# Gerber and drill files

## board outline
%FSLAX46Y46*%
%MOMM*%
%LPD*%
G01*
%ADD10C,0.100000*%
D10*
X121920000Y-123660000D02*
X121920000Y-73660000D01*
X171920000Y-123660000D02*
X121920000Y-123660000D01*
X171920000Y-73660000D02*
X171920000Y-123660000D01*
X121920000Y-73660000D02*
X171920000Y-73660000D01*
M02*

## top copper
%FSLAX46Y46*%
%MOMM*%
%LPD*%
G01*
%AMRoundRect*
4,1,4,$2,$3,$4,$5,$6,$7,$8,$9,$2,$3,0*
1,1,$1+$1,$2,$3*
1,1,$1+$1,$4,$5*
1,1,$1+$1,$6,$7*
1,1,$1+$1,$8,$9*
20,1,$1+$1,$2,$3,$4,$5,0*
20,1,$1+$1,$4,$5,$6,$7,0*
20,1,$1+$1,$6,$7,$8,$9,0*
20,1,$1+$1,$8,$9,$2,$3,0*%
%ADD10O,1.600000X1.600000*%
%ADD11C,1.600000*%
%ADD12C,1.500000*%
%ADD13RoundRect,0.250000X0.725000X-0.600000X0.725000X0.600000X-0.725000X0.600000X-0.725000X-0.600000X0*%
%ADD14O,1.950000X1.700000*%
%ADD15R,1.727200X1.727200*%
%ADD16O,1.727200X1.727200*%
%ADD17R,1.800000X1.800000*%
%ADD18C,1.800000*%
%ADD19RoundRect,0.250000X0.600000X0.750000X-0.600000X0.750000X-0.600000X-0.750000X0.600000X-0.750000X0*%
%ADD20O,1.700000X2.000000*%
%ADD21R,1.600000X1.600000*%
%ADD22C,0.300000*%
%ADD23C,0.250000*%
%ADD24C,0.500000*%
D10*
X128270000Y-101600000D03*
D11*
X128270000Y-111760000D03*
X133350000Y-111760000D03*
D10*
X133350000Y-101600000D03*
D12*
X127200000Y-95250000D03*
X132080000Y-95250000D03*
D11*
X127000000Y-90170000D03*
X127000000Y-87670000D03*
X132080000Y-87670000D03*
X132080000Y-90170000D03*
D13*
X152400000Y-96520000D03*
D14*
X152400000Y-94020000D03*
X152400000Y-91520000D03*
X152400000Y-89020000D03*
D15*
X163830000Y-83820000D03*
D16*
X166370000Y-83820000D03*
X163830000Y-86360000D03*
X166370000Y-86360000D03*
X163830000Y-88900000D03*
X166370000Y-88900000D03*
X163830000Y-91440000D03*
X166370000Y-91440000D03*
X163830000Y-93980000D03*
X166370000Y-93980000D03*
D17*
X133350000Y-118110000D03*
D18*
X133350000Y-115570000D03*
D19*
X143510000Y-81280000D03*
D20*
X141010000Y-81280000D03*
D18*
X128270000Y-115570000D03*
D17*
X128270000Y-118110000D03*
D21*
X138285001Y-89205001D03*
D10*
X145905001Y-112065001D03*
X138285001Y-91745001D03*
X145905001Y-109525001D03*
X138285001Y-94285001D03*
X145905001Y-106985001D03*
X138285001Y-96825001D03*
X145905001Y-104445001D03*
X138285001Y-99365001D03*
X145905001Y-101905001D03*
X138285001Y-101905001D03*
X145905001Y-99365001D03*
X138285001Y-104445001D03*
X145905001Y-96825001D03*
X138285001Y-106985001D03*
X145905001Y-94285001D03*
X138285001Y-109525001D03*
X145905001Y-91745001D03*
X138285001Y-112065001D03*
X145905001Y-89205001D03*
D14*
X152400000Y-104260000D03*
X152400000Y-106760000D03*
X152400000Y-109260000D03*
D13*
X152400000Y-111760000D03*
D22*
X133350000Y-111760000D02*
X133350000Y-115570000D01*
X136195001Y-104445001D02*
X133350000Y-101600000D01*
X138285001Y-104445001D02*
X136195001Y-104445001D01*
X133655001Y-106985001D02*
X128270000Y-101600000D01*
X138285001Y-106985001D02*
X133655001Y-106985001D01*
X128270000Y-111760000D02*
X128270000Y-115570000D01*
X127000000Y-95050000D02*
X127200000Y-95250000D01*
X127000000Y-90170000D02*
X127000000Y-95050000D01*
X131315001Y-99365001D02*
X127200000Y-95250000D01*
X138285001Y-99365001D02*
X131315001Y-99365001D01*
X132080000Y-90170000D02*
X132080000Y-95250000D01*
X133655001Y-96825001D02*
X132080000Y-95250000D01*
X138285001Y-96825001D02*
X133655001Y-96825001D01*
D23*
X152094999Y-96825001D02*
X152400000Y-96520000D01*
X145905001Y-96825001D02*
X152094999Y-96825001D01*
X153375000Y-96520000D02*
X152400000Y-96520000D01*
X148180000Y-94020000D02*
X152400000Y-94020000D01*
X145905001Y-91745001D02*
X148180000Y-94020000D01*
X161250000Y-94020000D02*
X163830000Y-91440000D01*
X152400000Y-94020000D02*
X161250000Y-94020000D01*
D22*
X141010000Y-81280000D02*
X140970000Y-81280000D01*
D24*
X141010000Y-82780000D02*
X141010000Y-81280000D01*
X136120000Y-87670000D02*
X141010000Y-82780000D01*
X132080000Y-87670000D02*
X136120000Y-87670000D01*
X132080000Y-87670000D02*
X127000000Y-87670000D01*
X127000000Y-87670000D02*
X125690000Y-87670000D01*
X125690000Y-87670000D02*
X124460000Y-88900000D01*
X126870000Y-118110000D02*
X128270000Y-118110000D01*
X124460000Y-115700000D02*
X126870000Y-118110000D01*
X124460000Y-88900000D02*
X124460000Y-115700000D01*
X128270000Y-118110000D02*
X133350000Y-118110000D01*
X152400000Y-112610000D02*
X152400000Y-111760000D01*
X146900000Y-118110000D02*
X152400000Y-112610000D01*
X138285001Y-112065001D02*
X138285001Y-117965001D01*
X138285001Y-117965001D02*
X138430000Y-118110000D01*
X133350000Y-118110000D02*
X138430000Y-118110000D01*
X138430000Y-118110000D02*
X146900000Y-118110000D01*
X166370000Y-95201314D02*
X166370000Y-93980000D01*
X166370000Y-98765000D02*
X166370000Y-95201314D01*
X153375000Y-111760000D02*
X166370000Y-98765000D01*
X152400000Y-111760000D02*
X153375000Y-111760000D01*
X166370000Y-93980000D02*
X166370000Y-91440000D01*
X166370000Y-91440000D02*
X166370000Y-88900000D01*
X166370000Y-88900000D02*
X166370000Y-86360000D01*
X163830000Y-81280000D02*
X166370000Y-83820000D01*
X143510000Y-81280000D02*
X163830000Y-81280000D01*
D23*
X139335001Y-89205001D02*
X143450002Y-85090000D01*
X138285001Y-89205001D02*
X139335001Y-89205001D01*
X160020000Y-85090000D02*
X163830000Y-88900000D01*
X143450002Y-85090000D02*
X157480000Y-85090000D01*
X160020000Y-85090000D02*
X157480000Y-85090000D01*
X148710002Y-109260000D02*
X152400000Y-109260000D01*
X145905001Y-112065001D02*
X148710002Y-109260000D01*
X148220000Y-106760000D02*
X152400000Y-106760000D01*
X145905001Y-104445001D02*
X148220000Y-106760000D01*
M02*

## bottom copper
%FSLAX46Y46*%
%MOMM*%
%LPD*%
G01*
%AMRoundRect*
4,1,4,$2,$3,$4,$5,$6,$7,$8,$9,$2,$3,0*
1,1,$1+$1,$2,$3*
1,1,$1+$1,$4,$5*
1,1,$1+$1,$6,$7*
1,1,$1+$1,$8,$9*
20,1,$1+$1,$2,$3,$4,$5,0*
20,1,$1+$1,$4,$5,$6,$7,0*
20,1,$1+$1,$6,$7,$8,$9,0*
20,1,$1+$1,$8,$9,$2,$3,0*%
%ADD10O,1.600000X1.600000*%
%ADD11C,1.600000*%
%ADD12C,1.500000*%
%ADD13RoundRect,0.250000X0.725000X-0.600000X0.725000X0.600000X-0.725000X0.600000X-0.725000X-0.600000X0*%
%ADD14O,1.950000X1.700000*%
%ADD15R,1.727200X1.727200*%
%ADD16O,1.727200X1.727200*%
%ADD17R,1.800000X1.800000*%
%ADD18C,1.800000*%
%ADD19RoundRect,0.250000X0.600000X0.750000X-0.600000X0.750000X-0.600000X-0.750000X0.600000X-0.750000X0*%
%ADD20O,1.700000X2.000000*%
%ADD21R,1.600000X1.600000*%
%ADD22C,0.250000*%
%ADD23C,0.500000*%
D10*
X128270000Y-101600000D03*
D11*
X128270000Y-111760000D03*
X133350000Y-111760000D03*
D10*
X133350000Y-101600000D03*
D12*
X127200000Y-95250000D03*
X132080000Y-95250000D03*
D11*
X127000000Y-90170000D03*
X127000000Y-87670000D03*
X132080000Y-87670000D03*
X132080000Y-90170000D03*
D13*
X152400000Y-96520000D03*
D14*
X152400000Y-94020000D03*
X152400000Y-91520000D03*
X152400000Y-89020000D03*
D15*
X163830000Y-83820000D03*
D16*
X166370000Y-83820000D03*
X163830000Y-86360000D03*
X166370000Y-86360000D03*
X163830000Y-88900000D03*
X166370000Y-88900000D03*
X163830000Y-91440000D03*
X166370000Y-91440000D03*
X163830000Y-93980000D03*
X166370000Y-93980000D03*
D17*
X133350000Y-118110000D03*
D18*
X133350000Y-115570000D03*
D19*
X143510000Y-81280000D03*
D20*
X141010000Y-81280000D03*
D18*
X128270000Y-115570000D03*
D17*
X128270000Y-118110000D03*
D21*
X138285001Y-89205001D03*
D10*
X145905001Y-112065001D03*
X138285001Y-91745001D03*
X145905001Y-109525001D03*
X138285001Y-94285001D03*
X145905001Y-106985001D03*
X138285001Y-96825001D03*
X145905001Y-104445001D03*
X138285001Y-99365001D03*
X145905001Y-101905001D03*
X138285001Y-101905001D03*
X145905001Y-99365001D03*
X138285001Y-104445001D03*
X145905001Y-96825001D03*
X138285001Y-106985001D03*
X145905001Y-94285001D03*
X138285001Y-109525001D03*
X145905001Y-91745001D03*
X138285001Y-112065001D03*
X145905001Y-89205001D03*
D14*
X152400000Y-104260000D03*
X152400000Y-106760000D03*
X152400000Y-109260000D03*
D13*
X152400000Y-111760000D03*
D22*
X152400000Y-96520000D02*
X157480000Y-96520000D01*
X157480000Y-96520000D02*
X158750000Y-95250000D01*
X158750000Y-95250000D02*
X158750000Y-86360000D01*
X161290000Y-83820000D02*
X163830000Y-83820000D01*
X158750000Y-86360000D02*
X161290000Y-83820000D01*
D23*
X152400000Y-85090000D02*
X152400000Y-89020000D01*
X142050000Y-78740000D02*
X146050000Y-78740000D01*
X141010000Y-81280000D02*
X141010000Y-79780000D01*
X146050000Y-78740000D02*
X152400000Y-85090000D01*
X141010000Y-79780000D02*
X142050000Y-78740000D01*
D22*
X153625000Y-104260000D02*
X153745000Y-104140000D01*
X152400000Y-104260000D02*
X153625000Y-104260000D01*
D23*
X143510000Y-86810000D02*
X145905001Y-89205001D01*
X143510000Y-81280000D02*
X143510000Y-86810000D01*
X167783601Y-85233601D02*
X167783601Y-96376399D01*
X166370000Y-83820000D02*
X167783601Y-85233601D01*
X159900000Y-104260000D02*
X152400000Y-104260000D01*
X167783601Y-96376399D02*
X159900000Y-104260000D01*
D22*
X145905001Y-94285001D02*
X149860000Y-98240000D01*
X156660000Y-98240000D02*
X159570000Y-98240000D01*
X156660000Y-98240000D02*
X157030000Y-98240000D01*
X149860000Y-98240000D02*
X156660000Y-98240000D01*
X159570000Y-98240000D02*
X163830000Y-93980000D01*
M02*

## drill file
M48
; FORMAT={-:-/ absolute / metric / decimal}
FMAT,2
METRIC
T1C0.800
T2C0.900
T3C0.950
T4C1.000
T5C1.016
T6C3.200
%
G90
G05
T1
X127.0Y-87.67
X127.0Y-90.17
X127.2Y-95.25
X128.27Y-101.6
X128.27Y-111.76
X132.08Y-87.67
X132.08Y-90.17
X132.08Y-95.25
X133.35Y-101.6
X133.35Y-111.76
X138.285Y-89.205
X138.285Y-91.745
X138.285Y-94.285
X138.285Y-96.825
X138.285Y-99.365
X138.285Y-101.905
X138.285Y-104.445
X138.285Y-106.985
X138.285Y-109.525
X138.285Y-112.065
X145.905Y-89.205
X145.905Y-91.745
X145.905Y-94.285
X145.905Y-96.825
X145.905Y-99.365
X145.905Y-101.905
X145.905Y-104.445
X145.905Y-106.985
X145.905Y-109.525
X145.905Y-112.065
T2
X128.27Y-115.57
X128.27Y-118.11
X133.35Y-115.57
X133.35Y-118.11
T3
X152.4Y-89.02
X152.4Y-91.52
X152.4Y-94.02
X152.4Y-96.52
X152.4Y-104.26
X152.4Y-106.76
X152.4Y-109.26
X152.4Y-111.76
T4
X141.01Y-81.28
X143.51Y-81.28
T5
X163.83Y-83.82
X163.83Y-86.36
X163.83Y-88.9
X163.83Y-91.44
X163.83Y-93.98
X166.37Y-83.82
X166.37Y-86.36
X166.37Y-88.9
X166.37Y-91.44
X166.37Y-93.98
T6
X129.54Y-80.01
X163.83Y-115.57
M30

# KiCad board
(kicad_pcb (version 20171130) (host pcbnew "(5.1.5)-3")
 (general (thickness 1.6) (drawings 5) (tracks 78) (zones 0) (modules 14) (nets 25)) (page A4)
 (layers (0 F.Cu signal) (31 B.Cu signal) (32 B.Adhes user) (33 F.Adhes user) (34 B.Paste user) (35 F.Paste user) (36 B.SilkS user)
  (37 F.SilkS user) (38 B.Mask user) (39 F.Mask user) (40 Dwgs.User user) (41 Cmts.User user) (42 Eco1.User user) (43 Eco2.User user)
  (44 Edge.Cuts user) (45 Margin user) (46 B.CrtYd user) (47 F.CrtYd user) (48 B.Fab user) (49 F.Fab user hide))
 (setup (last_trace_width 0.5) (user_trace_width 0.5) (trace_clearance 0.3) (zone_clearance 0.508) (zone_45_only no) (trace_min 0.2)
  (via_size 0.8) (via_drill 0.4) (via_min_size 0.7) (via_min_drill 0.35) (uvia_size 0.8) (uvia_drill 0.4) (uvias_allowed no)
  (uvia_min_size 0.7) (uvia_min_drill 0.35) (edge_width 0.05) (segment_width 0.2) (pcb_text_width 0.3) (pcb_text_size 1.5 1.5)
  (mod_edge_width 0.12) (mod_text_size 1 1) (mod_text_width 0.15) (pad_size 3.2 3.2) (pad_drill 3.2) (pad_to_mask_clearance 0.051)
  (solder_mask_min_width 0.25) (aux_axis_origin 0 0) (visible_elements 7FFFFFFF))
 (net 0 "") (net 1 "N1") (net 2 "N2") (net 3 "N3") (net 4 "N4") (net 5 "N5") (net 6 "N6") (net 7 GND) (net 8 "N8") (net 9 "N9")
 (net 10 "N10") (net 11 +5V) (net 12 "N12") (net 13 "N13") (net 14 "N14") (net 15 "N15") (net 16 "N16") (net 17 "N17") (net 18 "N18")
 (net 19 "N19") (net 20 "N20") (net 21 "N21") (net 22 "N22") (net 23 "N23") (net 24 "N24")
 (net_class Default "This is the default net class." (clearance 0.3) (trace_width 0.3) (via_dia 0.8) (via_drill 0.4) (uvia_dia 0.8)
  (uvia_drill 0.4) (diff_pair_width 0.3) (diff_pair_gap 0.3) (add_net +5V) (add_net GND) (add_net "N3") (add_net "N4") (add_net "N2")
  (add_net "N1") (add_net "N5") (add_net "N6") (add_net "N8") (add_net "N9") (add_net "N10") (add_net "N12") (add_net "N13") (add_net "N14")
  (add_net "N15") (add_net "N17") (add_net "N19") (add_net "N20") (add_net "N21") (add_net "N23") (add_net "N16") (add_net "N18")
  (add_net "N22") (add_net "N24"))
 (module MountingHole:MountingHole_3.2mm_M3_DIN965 (layer F.Cu) (at 163.83 115.57)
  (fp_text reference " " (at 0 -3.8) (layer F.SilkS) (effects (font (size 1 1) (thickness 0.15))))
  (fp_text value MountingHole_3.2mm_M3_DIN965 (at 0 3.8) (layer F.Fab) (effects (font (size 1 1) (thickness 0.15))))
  (pad 1 np_thru_hole circle (at 0 0) (size 3.2 3.2) (drill 3.2) (layers *.Cu *.Mask)))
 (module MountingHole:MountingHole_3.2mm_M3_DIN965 (layer F.Cu) (at 129.54 80.01)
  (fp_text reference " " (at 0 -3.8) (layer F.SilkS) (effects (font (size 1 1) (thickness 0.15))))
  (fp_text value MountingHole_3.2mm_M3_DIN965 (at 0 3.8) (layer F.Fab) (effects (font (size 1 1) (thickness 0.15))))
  (pad 1 np_thru_hole circle (at 0 0) (size 3.2 3.2) (drill 3.2) (layers *.Cu *.Mask)))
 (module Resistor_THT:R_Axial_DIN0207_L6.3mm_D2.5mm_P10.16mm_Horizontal (layer F.Cu) (at 128.27 111.76 90)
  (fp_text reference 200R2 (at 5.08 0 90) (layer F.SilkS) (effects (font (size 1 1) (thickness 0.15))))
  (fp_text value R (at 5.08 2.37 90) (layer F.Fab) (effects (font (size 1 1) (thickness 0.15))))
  (pad 2 thru_hole oval (at 10.16 0 90) (size 1.6 1.6) (drill 0.8) (layers *.Cu *.Mask) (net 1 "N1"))
  (pad 1 thru_hole circle (at 0 0 90) (size 1.6 1.6) (drill 0.8) (layers *.Cu *.Mask) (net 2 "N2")))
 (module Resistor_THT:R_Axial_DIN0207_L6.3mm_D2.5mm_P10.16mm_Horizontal (layer F.Cu) (at 133.35 111.76 90)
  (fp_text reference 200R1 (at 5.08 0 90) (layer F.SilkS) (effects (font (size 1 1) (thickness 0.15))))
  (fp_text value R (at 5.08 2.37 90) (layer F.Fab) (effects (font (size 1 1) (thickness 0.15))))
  (pad 1 thru_hole circle (at 0 0 90) (size 1.6 1.6) (drill 0.8) (layers *.Cu *.Mask) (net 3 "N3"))
  (pad 2 thru_hole oval (at 10.16 0 90) (size 1.6 1.6) (drill 0.8) (layers *.Cu *.Mask) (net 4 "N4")))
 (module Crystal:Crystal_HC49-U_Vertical (layer F.Cu) (at 127.2 95.25)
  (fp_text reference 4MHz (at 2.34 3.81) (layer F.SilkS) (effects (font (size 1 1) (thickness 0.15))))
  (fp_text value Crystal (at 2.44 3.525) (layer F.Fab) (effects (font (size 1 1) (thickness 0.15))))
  (pad 1 thru_hole circle (at 0 0) (size 1.5 1.5) (drill 0.8) (layers *.Cu *.Mask) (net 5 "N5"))
  (pad 2 thru_hole circle (at 4.88 0) (size 1.5 1.5) (drill 0.8) (layers *.Cu *.Mask) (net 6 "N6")))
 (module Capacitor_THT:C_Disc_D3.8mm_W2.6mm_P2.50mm (layer F.Cu) (at 127 90.17 90)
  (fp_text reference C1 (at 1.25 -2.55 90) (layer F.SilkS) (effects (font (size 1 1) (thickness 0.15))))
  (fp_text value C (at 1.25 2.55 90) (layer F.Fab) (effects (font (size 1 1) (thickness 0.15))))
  (pad 1 thru_hole circle (at 0 0 90) (size 1.6 1.6) (drill 0.8) (layers *.Cu *.Mask) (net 5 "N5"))
  (pad 2 thru_hole circle (at 2.5 0 90) (size 1.6 1.6) (drill 0.8) (layers *.Cu *.Mask) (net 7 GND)))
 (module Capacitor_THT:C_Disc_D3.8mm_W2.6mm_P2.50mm (layer F.Cu) (at 132.08 90.17 90)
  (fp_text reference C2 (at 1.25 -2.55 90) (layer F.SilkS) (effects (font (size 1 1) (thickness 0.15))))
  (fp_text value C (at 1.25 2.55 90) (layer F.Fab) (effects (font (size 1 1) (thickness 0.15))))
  (pad 2 thru_hole circle (at 2.5 0 90) (size 1.6 1.6) (drill 0.8) (layers *.Cu *.Mask) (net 7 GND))
  (pad 1 thru_hole circle (at 0 0 90) (size 1.6 1.6) (drill 0.8) (layers *.Cu *.Mask) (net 6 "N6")))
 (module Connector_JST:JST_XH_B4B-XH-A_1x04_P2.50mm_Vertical (layer F.Cu) (at 152.4 96.52 90)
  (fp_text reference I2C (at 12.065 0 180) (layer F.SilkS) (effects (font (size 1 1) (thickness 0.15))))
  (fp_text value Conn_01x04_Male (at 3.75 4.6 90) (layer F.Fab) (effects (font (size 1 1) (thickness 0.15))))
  (pad 1 thru_hole roundrect (at 0 0 90) (size 1.7 1.95) (drill 0.95) (layers *.Cu *.Mask) (roundrect_rratio 0.147059) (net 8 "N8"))
  (pad 2 thru_hole oval (at 2.5 0 90) (size 1.7 1.95) (drill 0.95) (layers *.Cu *.Mask) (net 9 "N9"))
  (pad 3 thru_hole oval (at 5 0 90) (size 1.7 1.95) (drill 0.95) (layers *.Cu *.Mask) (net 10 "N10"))
  (pad 4 thru_hole oval (at 7.5 0 90) (size 1.7 1.95) (drill 0.95) (layers *.Cu *.Mask) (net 7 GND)))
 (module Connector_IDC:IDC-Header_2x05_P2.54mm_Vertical (layer F.Cu) (at 163.83 83.82)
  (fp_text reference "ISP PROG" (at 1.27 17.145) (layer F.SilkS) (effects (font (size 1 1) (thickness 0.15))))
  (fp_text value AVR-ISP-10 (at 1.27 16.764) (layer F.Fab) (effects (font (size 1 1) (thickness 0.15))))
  (pad 1 thru_hole rect (at 0 0) (size 1.7272 1.7272) (drill 1.016) (layers *.Cu *.Mask) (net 8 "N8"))
  (pad 2 thru_hole oval (at 2.54 0) (size 1.7272 1.7272) (drill 1.016) (layers *.Cu *.Mask) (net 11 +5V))
  (pad 3 thru_hole oval (at 0 2.54) (size 1.7272 1.7272) (drill 1.016) (layers *.Cu *.Mask) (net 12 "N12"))
  (pad 4 thru_hole oval (at 2.54 2.54) (size 1.7272 1.7272) (drill 1.016) (layers *.Cu *.Mask) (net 7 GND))
  (pad 5 thru_hole oval (at 0 5.08) (size 1.7272 1.7272) (drill 1.016) (layers *.Cu *.Mask) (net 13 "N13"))
  (pad 6 thru_hole oval (at 2.54 5.08) (size 1.7272 1.7272) (drill 1.016) (layers *.Cu *.Mask) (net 7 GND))
  (pad 7 thru_hole oval (at 0 7.62) (size 1.7272 1.7272) (drill 1.016) (layers *.Cu *.Mask) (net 9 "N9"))
  (pad 8 thru_hole oval (at 2.54 7.62) (size 1.7272 1.7272) (drill 1.016) (layers *.Cu *.Mask) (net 7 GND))
  (pad 9 thru_hole oval (at 0 10.16) (size 1.7272 1.7272) (drill 1.016) (layers *.Cu *.Mask) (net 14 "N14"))
  (pad 10 thru_hole oval (at 2.54 10.16) (size 1.7272 1.7272) (drill 1.016) (layers *.Cu *.Mask) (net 7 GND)))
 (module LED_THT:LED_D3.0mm (layer F.Cu) (at 133.35 118.11 90)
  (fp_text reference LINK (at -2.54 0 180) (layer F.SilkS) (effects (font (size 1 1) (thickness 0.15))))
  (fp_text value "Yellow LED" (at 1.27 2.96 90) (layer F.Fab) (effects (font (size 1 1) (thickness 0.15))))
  (pad 1 thru_hole rect (at 0 0 90) (size 1.8 1.8) (drill 0.9) (layers *.Cu *.Mask) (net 7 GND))
  (pad 2 thru_hole circle (at 2.54 0 90) (size 1.8 1.8) (drill 0.9) (layers *.Cu *.Mask) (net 3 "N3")))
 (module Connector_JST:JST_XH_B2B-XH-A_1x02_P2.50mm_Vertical (layer F.Cu) (at 143.51 81.28 180)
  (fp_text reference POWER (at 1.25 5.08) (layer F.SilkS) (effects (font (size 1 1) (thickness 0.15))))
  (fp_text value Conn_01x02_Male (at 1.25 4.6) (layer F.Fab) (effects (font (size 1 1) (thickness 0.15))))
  (pad 1 thru_hole roundrect (at 0 0 180) (size 1.7 2) (drill 1) (layers *.Cu *.Mask) (roundrect_rratio 0.147059) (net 11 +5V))
  (pad 2 thru_hole oval (at 2.5 0 180) (size 1.7 2) (drill 1) (layers *.Cu *.Mask) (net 7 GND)))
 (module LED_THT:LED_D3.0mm (layer F.Cu) (at 128.27 118.11 90)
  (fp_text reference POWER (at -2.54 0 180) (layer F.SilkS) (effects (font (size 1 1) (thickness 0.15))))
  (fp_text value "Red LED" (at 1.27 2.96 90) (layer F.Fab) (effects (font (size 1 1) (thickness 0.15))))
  (pad 2 thru_hole circle (at 2.54 0 90) (size 1.8 1.8) (drill 0.9) (layers *.Cu *.Mask) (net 2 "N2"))
  (pad 1 thru_hole rect (at 0 0 90) (size 1.8 1.8) (drill 0.9) (layers *.Cu *.Mask) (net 7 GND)))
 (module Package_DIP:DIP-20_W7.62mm (layer F.Cu) (at 138.285001 89.205001)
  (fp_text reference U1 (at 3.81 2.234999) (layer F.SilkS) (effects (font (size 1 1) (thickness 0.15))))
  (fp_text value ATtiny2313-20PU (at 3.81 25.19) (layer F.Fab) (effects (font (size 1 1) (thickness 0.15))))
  (pad 1 thru_hole rect (at 0 0) (size 1.6 1.6) (drill 0.8) (layers *.Cu *.Mask) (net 13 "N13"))
  (pad 11 thru_hole oval (at 7.62 22.86) (size 1.6 1.6) (drill 0.8) (layers *.Cu *.Mask) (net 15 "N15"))
  (pad 2 thru_hole oval (at 0 2.54) (size 1.6 1.6) (drill 0.8) (layers *.Cu *.Mask) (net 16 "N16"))
  (pad 12 thru_hole oval (at 7.62 20.32) (size 1.6 1.6) (drill 0.8) (layers *.Cu *.Mask) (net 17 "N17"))
  (pad 3 thru_hole oval (at 0 5.08) (size 1.6 1.6) (drill 0.8) (layers *.Cu *.Mask) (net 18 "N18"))
  (pad 13 thru_hole oval (at 7.62 17.78) (size 1.6 1.6) (drill 0.8) (layers *.Cu *.Mask) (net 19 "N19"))
  (pad 4 thru_hole oval (at 0 7.62) (size 1.6 1.6) (drill 0.8) (layers *.Cu *.Mask) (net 6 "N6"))
  (pad 14 thru_hole oval (at 7.62 15.24) (size 1.6 1.6) (drill 0.8) (layers *.Cu *.Mask) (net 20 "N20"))
  (pad 5 thru_hole oval (at 0 10.16) (size 1.6 1.6) (drill 0.8) (layers *.Cu *.Mask) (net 5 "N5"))
  (pad 15 thru_hole oval (at 7.62 12.7) (size 1.6 1.6) (drill 0.8) (layers *.Cu *.Mask) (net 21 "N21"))
  (pad 6 thru_hole oval (at 0 12.7) (size 1.6 1.6) (drill 0.8) (layers *.Cu *.Mask) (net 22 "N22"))
  (pad 16 thru_hole oval (at 7.62 10.16) (size 1.6 1.6) (drill 0.8) (layers *.Cu *.Mask) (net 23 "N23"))
  (pad 7 thru_hole oval (at 0 15.24) (size 1.6 1.6) (drill 0.8) (layers *.Cu *.Mask) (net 4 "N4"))
  (pad 17 thru_hole oval (at 7.62 7.62) (size 1.6 1.6) (drill 0.8) (layers *.Cu *.Mask) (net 8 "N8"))
  (pad 8 thru_hole oval (at 0 17.78) (size 1.6 1.6) (drill 0.8) (layers *.Cu *.Mask) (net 1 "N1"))
  (pad 18 thru_hole oval (at 7.62 5.08) (size 1.6 1.6) (drill 0.8) (layers *.Cu *.Mask) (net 14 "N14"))
  (pad 9 thru_hole oval (at 0 20.32) (size 1.6 1.6) (drill 0.8) (layers *.Cu *.Mask) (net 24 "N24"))
  (pad 19 thru_hole oval (at 7.62 2.54) (size 1.6 1.6) (drill 0.8) (layers *.Cu *.Mask) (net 9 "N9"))
  (pad 10 thru_hole oval (at 0 22.86) (size 1.6 1.6) (drill 0.8) (layers *.Cu *.Mask) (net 7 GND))
  (pad 20 thru_hole oval (at 7.62 0) (size 1.6 1.6) (drill 0.8) (layers *.Cu *.Mask) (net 11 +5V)))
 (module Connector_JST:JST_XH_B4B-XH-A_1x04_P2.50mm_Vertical (layer F.Cu) (at 152.4 111.76 90)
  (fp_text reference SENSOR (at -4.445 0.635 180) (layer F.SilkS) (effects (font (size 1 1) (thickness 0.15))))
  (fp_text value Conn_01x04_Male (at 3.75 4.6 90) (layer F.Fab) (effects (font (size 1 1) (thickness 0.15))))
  (pad 4 thru_hole oval (at 7.5 0 90) (size 1.7 1.95) (drill 0.95) (layers *.Cu *.Mask) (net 11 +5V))
  (pad 3 thru_hole oval (at 5 0 90) (size 1.7 1.95) (drill 0.95) (layers *.Cu *.Mask) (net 20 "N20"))
  (pad 2 thru_hole oval (at 2.5 0 90) (size 1.7 1.95) (drill 0.95) (layers *.Cu *.Mask) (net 15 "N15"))
  (pad 1 thru_hole roundrect (at 0 0 90) (size 1.7 1.95) (drill 0.95) (layers *.Cu *.Mask) (roundrect_rratio 0.147059) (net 7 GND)))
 (gr_line (start 121.92 123.66) (end 121.92 73.66) (layer Edge.Cuts) (width 0.1))
 (gr_line (start 171.92 123.66) (end 121.92 123.66) (layer Edge.Cuts) (width 0.1))
 (gr_line (start 171.92 73.66) (end 171.92 123.66) (layer Edge.Cuts) (width 0.1))
 (gr_line (start 121.92 73.66) (end 171.92 73.66) (layer Edge.Cuts) (width 0.1))
 (segment (start 133.35 111.76) (end 133.35 115.57) (width 0.3) (layer F.Cu) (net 3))
 (segment (start 136.195001 104.445001) (end 133.35 101.6) (width 0.3) (layer F.Cu) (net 4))
 (segment (start 138.285001 104.445001) (end 136.195001 104.445001) (width 0.3) (layer F.Cu) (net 4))
 (segment (start 133.655001 106.985001) (end 128.27 101.6) (width 0.3) (layer F.Cu) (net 1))
 (segment (start 138.285001 106.985001) (end 133.655001 106.985001) (width 0.3) (layer F.Cu) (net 1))
 (segment (start 128.27 111.76) (end 128.27 115.57) (width 0.3) (layer F.Cu) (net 2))
 (segment (start 127 95.05) (end 127.2 95.25) (width 0.3) (layer F.Cu) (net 5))
 (segment (start 127 90.17) (end 127 95.05) (width 0.3) (layer F.Cu) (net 5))
 (segment (start 131.315001 99.365001) (end 127.2 95.25) (width 0.3) (layer F.Cu) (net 5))
 (segment (start 138.285001 99.365001) (end 131.315001 99.365001) (width 0.3) (layer F.Cu) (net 5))
 (segment (start 132.08 90.17) (end 132.08 95.25) (width 0.3) (layer F.Cu) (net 6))
 (segment (start 133.655001 96.825001) (end 132.08 95.25) (width 0.3) (layer F.Cu) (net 6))
 (segment (start 138.285001 96.825001) (end 133.655001 96.825001) (width 0.3) (layer F.Cu) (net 6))
 (segment (start 152.094999 96.825001) (end 152.4 96.52) (width 0.25) (layer F.Cu) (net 8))
 (segment (start 145.905001 96.825001) (end 152.094999 96.825001) (width 0.25) (layer F.Cu) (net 8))
 (segment (start 153.375 96.52) (end 152.4 96.52) (width 0.25) (layer F.Cu) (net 8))
 (segment (start 152.4 96.52) (end 157.48 96.52) (width 0.25) (layer B.Cu) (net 8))
 (segment (start 157.48 96.52) (end 158.75 95.25) (width 0.25) (layer B.Cu) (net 8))
 (segment (start 158.75 95.25) (end 158.75 86.36) (width 0.25) (layer B.Cu) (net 8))
 (segment (start 161.29 83.82) (end 163.83 83.82) (width 0.25) (layer B.Cu) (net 8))
 (segment (start 158.75 86.36) (end 161.29 83.82) (width 0.25) (layer B.Cu) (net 8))
 (segment (start 148.18 94.02) (end 152.4 94.02) (width 0.25) (layer F.Cu) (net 9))
 (segment (start 145.905001 91.745001) (end 148.18 94.02) (width 0.25) (layer F.Cu) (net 9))
 (segment (start 161.25 94.02) (end 163.83 91.44) (width 0.25) (layer F.Cu) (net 9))
 (segment (start 152.4 94.02) (end 161.25 94.02) (width 0.25) (layer F.Cu) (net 9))
 (segment (start 141.01 81.28) (end 140.97 81.28) (width 0.3) (layer F.Cu) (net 7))
 (segment (start 141.01 82.78) (end 141.01 81.28) (width 0.5) (layer F.Cu) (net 7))
 (segment (start 136.12 87.67) (end 141.01 82.78) (width 0.5) (layer F.Cu) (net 7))
 (segment (start 132.08 87.67) (end 136.12 87.67) (width 0.5) (layer F.Cu) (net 7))
 (segment (start 132.08 87.67) (end 127 87.67) (width 0.5) (layer F.Cu) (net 7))
 (segment (start 127 87.67) (end 125.69 87.67) (width 0.5) (layer F.Cu) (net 7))
 (segment (start 125.69 87.67) (end 124.46 88.9) (width 0.5) (layer F.Cu) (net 7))
 (segment (start 126.87 118.11) (end 128.27 118.11) (width 0.5) (layer F.Cu) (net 7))
 (segment (start 124.46 115.7) (end 126.87 118.11) (width 0.5) (layer F.Cu) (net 7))
 (segment (start 124.46 88.9) (end 124.46 115.7) (width 0.5) (layer F.Cu) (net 7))
 (segment (start 128.27 118.11) (end 133.35 118.11) (width 0.5) (layer F.Cu) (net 7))
 (segment (start 152.4 112.61) (end 152.4 111.76) (width 0.5) (layer F.Cu) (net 7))
 (segment (start 146.9 118.11) (end 152.4 112.61) (width 0.5) (layer F.Cu) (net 7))
 (segment (start 138.285001 112.065001) (end 138.285001 117.965001) (width 0.5) (layer F.Cu) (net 7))
 (segment (start 138.285001 117.965001) (end 138.43 118.11) (width 0.5) (layer F.Cu) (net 7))
 (segment (start 133.35 118.11) (end 138.43 118.11) (width 0.5) (layer F.Cu) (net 7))
 (segment (start 138.43 118.11) (end 146.9 118.11) (width 0.5) (layer F.Cu) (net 7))
 (segment (start 166.37 95.201314) (end 166.37 93.98) (width 0.5) (layer F.Cu) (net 7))
 (segment (start 166.37 98.765) (end 166.37 95.201314) (width 0.5) (layer F.Cu) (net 7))
 (segment (start 153.375 111.76) (end 166.37 98.765) (width 0.5) (layer F.Cu) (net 7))
 (segment (start 152.4 111.76) (end 153.375 111.76) (width 0.5) (layer F.Cu) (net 7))
 (segment (start 166.37 93.98) (end 166.37 91.44) (width 0.5) (layer F.Cu) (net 7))
 (segment (start 166.37 91.44) (end 166.37 88.9) (width 0.5) (layer F.Cu) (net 7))
 (segment (start 166.37 88.9) (end 166.37 86.36) (width 0.5) (layer F.Cu) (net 7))
 (segment (start 152.4 85.09) (end 152.4 89.02) (width 0.5) (layer B.Cu) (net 7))
 (segment (start 142.05 78.74) (end 146.05 78.74) (width 0.5) (layer B.Cu) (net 7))
 (segment (start 141.01 81.28) (end 141.01 79.78) (width 0.5) (layer B.Cu) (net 7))
 (segment (start 146.05 78.74) (end 152.4 85.09) (width 0.5) (layer B.Cu) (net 7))
 (segment (start 141.01 79.78) (end 142.05 78.74) (width 0.5) (layer B.Cu) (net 7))
 (segment (start 153.625 104.26) (end 153.745 104.14) (width 0.25) (layer B.Cu) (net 11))
 (segment (start 152.4 104.26) (end 153.625 104.26) (width 0.25) (layer B.Cu) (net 11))
 (segment (start 163.83 81.28) (end 166.37 83.82) (width 0.5) (layer F.Cu) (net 11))
 (segment (start 143.51 81.28) (end 163.83 81.28) (width 0.5) (layer F.Cu) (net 11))
 (segment (start 143.51 86.81) (end 145.905001 89.205001) (width 0.5) (layer B.Cu) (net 11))
 (segment (start 143.51 81.28) (end 143.51 86.81) (width 0.5) (layer B.Cu) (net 11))
 (segment (start 167.783601 85.233601) (end 167.783601 96.376399) (width 0.5) (layer B.Cu) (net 11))
 (segment (start 166.37 83.82) (end 167.783601 85.233601) (width 0.5) (layer B.Cu) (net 11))
 (segment (start 159.9 104.26) (end 152.4 104.26) (width 0.5) (layer B.Cu) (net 11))
 (segment (start 167.783601 96.376399) (end 159.9 104.26) (width 0.5) (layer B.Cu) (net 11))
 (segment (start 139.335001 89.205001) (end 143.450002 85.09) (width 0.25) (layer F.Cu) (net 13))
 (segment (start 138.285001 89.205001) (end 139.335001 89.205001) (width 0.25) (layer F.Cu) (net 13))
 (segment (start 160.02 85.09) (end 163.83 88.9) (width 0.25) (layer F.Cu) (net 13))
 (segment (start 143.450002 85.09) (end 157.48 85.09) (width 0.25) (layer F.Cu) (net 13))
 (segment (start 160.02 85.09) (end 157.48 85.09) (width 0.25) (layer F.Cu) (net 13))
 (segment (start 145.905001 94.285001) (end 149.86 98.24) (width 0.25) (layer B.Cu) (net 14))
 (segment (start 156.66 98.24) (end 159.57 98.24) (width 0.25) (layer B.Cu) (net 14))
 (segment (start 156.66 98.24) (end 157.03 98.24) (width 0.25) (layer B.Cu) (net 14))
 (segment (start 149.86 98.24) (end 156.66 98.24) (width 0.25) (layer B.Cu) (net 14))
 (segment (start 159.57 98.24) (end 163.83 93.98) (width 0.25) (layer B.Cu) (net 14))
 (segment (start 148.710002 109.26) (end 152.4 109.26) (width 0.25) (layer F.Cu) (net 15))
 (segment (start 145.905001 112.065001) (end 148.710002 109.26) (width 0.25) (layer F.Cu) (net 15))
 (segment (start 148.22 106.76) (end 152.4 106.76) (width 0.25) (layer F.Cu) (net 20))
 (segment (start 145.905001 104.445001) (end 148.22 106.76) (width 0.25) (layer F.Cu) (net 20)))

